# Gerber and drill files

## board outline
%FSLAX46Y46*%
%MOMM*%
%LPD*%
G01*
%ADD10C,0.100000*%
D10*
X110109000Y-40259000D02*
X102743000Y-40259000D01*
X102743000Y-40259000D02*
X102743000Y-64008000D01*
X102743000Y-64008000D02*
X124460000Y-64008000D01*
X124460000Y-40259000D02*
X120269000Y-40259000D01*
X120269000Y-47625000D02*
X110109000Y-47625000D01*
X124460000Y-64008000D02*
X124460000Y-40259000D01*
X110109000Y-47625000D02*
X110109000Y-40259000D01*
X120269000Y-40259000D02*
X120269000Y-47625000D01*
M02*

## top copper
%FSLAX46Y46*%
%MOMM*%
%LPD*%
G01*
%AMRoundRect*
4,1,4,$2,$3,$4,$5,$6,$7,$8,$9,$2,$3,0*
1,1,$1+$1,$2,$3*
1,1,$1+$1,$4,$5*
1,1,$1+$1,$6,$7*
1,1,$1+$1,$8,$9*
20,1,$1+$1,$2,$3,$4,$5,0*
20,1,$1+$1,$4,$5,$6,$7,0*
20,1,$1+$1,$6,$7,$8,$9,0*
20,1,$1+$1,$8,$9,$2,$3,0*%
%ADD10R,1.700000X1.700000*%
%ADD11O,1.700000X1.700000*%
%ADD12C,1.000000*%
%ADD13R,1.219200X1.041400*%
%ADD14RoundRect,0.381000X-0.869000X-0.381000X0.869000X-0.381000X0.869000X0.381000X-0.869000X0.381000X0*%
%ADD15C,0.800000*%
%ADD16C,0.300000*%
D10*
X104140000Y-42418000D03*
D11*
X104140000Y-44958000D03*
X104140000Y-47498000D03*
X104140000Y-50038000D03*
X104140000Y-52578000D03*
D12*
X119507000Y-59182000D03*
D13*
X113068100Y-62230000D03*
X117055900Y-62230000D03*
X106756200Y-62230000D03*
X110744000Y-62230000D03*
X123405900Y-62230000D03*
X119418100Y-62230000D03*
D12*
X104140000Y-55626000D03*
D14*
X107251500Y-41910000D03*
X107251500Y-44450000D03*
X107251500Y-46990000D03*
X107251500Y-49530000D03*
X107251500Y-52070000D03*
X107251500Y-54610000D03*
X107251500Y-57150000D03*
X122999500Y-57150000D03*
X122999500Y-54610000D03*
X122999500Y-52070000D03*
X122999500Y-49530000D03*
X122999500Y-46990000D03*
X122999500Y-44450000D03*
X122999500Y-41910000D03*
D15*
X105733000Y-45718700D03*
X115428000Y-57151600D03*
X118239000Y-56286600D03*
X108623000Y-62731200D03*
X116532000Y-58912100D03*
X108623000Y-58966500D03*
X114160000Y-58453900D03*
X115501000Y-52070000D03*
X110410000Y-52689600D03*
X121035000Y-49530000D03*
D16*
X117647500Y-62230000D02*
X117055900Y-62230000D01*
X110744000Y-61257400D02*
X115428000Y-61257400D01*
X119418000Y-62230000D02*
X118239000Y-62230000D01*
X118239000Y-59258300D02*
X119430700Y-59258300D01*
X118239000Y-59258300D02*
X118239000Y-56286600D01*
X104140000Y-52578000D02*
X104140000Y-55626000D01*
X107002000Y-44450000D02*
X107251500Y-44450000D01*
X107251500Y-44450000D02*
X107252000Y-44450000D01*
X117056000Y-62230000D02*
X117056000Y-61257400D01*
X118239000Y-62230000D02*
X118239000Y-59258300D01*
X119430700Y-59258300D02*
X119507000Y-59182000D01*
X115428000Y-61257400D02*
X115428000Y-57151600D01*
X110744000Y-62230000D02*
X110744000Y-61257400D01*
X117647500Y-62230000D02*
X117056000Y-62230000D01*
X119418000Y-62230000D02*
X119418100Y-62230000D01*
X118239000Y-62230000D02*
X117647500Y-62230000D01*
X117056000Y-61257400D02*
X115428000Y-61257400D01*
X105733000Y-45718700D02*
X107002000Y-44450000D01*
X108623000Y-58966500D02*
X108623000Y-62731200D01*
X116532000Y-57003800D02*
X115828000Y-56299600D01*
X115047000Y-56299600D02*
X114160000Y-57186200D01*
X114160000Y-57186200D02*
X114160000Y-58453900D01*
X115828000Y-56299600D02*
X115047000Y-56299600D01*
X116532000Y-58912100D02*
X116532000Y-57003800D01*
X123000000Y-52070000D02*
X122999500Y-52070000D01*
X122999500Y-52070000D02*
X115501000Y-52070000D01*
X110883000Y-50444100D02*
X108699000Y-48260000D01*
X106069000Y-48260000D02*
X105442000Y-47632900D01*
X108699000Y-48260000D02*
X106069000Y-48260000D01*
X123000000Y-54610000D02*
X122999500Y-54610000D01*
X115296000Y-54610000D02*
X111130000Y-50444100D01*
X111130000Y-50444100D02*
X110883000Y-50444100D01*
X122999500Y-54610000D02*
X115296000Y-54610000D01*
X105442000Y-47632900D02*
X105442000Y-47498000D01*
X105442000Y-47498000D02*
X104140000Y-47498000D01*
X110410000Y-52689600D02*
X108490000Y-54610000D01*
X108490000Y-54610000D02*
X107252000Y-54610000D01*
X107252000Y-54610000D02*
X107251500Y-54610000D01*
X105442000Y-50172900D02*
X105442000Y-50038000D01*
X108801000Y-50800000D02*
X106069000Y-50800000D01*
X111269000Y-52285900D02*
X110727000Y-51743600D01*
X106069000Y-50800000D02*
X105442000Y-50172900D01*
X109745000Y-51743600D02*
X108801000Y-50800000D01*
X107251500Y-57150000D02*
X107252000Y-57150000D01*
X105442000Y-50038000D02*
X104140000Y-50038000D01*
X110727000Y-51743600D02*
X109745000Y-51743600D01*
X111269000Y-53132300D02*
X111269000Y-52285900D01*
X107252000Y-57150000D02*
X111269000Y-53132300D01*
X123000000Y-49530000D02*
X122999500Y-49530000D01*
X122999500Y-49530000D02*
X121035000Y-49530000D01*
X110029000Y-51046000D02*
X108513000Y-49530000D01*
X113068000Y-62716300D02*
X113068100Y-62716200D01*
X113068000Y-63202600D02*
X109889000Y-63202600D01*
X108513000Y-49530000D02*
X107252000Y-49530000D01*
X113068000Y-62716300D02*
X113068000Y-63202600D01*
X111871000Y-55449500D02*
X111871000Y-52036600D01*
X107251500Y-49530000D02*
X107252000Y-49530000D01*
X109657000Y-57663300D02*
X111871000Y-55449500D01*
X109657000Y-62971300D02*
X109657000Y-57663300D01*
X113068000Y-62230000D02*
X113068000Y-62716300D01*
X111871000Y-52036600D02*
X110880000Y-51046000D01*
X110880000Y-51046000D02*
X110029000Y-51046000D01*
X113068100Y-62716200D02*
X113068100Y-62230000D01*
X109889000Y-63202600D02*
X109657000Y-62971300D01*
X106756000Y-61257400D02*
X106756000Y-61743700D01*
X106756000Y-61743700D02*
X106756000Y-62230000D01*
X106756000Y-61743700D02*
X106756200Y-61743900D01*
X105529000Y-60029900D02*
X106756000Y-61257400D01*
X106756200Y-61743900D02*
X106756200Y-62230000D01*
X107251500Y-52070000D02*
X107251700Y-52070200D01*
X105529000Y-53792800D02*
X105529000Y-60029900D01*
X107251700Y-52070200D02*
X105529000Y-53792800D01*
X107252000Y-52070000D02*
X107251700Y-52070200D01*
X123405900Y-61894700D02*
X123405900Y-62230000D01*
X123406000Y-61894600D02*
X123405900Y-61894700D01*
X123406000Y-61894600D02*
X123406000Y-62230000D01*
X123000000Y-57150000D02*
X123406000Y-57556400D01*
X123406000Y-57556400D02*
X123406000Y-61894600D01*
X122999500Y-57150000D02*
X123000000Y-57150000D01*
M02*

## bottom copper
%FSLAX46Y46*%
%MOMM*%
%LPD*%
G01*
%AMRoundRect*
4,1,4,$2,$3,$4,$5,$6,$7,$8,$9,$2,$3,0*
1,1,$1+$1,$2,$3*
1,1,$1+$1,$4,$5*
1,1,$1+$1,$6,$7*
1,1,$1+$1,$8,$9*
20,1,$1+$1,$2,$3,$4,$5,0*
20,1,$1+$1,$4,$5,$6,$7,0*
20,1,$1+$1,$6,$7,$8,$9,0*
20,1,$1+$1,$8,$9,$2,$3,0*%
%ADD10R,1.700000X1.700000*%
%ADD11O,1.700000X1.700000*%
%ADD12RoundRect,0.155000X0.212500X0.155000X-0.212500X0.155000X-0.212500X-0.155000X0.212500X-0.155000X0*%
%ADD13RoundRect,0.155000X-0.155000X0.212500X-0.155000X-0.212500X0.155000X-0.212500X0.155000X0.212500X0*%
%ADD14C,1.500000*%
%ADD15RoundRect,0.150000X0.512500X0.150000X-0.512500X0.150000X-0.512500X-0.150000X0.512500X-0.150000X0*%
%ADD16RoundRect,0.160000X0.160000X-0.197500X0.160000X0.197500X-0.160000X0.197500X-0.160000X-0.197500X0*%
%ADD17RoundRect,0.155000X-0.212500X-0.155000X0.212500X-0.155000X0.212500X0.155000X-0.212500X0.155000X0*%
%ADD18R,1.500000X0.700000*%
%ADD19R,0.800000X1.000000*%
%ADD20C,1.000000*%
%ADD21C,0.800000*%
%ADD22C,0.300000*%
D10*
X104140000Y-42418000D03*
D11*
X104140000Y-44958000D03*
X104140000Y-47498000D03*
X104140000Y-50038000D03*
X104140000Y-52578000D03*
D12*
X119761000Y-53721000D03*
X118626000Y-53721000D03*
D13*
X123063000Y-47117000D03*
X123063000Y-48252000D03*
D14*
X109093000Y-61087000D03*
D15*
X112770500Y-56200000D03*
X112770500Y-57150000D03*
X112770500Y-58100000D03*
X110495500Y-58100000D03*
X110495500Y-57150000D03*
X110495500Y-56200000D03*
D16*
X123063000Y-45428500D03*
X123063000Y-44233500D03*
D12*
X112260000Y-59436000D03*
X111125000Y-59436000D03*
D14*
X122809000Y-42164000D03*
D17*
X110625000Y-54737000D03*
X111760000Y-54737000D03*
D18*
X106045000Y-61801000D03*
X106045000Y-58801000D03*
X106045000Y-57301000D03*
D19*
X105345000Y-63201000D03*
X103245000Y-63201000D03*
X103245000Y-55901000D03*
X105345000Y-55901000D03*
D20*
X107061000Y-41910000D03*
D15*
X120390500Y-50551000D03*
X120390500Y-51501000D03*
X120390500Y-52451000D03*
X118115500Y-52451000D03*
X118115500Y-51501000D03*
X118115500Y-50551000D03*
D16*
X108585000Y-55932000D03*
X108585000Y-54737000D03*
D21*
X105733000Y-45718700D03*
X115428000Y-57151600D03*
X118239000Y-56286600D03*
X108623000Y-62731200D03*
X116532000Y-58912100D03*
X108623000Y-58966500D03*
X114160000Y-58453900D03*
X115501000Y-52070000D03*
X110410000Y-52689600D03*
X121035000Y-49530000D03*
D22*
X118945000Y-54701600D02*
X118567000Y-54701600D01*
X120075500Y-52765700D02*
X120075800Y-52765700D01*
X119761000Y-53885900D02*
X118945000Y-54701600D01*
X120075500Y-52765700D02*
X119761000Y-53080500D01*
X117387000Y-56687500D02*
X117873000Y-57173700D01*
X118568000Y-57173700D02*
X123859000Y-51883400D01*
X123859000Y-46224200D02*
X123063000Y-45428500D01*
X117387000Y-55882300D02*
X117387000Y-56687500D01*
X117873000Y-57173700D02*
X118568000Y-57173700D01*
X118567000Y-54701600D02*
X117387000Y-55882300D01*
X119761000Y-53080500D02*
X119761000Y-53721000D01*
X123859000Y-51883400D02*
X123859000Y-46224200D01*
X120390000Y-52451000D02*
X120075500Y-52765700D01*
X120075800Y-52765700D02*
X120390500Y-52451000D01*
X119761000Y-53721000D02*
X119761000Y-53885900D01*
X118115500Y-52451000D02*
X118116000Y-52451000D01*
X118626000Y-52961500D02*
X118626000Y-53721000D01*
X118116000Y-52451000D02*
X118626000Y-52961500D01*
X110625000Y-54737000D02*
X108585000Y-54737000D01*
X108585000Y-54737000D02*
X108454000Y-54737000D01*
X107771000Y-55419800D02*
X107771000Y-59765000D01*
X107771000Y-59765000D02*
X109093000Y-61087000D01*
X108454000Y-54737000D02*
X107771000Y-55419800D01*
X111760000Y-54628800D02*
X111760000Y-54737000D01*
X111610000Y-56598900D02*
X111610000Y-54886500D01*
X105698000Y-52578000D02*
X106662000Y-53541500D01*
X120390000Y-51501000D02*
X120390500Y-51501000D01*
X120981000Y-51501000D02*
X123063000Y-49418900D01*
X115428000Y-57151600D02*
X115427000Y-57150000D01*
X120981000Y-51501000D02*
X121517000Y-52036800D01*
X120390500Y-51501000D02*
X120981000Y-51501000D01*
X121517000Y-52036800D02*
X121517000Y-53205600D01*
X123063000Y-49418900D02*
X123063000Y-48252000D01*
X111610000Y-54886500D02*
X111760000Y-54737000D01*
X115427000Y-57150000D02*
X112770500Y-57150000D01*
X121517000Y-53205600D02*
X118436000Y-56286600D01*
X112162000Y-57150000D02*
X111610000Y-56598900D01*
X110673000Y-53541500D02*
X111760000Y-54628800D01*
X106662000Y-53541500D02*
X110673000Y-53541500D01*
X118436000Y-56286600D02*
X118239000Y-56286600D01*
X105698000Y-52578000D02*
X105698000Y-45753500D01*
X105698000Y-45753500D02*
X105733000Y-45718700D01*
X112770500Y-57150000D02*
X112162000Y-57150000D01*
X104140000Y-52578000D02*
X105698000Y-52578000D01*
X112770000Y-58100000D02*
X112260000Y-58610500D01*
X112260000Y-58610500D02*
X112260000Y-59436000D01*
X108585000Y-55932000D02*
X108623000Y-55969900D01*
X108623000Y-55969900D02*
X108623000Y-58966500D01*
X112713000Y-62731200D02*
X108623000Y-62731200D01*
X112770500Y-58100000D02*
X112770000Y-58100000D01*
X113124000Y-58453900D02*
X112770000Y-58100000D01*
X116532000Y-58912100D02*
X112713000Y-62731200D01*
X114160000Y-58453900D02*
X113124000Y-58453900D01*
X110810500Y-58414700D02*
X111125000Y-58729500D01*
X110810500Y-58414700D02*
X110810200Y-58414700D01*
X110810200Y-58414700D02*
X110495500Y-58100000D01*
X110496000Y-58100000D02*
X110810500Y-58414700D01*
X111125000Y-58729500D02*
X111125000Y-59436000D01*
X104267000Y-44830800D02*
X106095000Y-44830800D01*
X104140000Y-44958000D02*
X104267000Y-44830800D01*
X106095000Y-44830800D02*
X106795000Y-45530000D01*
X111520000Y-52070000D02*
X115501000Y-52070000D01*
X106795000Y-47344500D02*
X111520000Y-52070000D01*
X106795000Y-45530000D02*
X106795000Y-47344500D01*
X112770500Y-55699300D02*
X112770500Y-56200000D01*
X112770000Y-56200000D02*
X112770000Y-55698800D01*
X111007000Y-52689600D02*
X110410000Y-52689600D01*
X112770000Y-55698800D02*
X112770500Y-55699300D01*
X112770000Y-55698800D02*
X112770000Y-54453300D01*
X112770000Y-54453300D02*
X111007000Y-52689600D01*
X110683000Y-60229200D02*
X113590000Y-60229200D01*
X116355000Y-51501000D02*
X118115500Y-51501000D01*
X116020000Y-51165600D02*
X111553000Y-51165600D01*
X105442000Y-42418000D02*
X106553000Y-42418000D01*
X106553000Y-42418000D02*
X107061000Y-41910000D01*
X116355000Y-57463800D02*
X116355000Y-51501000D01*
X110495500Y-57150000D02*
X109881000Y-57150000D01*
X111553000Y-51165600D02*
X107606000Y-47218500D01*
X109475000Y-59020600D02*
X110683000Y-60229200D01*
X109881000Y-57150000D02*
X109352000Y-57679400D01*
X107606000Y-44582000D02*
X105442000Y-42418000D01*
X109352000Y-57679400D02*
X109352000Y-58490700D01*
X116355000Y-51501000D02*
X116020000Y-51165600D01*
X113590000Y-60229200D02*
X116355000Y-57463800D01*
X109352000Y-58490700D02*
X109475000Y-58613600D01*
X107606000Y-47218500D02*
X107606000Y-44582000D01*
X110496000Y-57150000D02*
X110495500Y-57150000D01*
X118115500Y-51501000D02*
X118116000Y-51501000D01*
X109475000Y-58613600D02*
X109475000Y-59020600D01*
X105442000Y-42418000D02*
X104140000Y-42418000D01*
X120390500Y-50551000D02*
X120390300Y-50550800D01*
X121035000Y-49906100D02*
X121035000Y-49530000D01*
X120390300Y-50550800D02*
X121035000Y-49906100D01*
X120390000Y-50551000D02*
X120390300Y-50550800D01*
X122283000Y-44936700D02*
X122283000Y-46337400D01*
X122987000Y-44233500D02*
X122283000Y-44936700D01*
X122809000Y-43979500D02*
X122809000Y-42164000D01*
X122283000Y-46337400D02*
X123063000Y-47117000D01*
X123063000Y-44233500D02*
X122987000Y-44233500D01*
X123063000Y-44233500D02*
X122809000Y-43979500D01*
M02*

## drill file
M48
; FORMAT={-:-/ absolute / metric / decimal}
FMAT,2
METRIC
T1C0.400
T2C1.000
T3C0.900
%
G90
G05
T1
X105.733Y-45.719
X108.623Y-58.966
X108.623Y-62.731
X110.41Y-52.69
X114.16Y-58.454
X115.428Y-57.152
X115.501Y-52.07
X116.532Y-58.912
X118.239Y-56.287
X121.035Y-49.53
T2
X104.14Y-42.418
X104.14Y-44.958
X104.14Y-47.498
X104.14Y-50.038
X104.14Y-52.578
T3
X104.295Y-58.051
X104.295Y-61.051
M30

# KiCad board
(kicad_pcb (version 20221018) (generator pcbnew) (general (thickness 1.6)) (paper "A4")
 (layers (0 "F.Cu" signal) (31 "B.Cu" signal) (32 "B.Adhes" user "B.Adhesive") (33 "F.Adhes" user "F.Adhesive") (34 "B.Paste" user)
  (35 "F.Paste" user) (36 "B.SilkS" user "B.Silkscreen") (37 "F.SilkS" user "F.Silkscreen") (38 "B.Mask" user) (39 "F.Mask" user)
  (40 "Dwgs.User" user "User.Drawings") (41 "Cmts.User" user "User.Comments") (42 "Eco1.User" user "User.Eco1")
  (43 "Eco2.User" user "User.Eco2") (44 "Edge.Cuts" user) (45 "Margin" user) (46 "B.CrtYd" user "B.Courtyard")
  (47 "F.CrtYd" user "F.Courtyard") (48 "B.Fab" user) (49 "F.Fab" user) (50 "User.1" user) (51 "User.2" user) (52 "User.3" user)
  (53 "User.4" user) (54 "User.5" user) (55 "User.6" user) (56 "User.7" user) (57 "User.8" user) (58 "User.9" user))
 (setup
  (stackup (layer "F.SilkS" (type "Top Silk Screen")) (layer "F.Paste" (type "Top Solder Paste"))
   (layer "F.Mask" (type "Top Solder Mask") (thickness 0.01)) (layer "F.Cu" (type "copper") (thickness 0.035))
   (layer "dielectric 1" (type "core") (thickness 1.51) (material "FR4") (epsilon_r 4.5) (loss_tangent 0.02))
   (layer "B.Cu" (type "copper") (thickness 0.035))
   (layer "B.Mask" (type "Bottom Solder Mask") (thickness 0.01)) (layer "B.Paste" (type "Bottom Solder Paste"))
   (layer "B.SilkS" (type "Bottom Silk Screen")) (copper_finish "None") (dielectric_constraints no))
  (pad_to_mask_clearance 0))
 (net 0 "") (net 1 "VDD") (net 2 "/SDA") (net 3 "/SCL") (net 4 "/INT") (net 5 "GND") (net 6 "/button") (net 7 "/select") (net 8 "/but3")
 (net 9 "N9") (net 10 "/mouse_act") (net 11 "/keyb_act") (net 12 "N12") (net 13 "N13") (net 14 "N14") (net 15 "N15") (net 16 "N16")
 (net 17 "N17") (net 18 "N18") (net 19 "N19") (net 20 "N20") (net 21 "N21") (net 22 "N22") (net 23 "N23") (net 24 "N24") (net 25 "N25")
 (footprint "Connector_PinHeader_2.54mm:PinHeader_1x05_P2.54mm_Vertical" (layer "F.Cu") (at 104.14 42.418)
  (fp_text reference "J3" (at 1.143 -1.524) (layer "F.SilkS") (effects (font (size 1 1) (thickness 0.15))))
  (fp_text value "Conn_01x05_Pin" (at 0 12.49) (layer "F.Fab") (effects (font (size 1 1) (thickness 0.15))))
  (pad "1" thru_hole rect (at 0 0) (size 1.7 1.7) (drill 1) (layers "*.Cu" "*.Mask") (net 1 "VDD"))
  (pad "2" thru_hole oval (at 0 2.54) (size 1.7 1.7) (drill 1) (layers "*.Cu" "*.Mask") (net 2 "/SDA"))
  (pad "3" thru_hole oval (at 0 5.08) (size 1.7 1.7) (drill 1) (layers "*.Cu" "*.Mask") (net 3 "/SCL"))
  (pad "4" thru_hole oval (at 0 7.62) (size 1.7 1.7) (drill 1) (layers "*.Cu" "*.Mask") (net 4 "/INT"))
  (pad "5" thru_hole oval (at 0 10.16) (size 1.7 1.7) (drill 1) (layers "*.Cu" "*.Mask") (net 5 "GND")))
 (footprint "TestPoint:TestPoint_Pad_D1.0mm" (layer "F.Cu") (at 119.507 59.182)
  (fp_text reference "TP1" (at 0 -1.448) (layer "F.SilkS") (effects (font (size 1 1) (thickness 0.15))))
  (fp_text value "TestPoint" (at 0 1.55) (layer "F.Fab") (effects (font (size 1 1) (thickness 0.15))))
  (pad "1" smd circle (at 0 0) (size 1 1) (layers "F.Cu" "F.Mask") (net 5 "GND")))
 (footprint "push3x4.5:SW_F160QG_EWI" (layer "F.Cu") (at 115.062 62.23)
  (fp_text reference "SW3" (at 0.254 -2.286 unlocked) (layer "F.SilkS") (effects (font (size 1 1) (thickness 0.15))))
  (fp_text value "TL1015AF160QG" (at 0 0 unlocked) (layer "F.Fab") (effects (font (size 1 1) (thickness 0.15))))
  (pad "1" smd rect (at -1.9939 0) (size 1.2192 1.0414) (layers "F.Cu" "F.Paste" "F.Mask") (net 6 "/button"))
  (pad "2" smd rect (at 1.9939 0) (size 1.2192 1.0414) (layers "F.Cu" "F.Paste" "F.Mask") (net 5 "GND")))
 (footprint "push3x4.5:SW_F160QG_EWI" (layer "F.Cu") (at 108.7501 62.23)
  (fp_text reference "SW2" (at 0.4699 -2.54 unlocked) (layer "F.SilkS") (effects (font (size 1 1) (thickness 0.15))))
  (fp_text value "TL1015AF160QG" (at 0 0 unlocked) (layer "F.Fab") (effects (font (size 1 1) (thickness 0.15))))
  (pad "1" smd rect (at -1.9939 0) (size 1.2192 1.0414) (layers "F.Cu" "F.Paste" "F.Mask") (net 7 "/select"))
  (pad "2" smd rect (at 1.9939 0) (size 1.2192 1.0414) (layers "F.Cu" "F.Paste" "F.Mask") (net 5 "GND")))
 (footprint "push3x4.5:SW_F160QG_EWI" (layer "F.Cu") (at 121.412 62.23 180)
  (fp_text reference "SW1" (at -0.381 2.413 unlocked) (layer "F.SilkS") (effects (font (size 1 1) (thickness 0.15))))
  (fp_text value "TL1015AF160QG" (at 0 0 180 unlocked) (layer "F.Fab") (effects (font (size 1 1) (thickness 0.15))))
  (pad "1" smd rect (at -1.9939 0 180) (size 1.2192 1.0414) (layers "F.Cu" "F.Paste" "F.Mask") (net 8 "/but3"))
  (pad "2" smd rect (at 1.9939 0 180) (size 1.2192 1.0414) (layers "F.Cu" "F.Paste" "F.Mask") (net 5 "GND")))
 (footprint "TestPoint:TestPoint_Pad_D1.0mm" (layer "F.Cu") (at 104.14 55.626)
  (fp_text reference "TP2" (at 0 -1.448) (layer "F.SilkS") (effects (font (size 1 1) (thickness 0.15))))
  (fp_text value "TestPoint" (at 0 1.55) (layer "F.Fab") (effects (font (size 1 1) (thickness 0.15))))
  (pad "1" smd circle (at 0 0) (size 1 1) (layers "F.Cu" "F.Mask") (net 5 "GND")))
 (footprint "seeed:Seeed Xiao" (layer "F.Cu") (at 109.0295 41.91)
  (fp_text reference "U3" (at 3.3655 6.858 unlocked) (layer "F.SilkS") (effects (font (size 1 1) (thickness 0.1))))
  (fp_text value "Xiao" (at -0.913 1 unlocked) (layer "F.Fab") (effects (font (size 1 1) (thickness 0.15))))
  (pad "1" smd roundrect (at -1.778 0) (size 2.5 1.524) (layers "F.Cu" "F.Paste" "F.Mask") (roundrect_rratio 0.25) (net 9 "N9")
   (thermal_bridge_angle 45))
  (pad "2" smd roundrect (at -1.778 2.54) (size 2.5 1.524) (layers "F.Cu" "F.Paste" "F.Mask") (roundrect_rratio 0.25) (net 5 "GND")
   (thermal_bridge_angle 45))
  (pad "3" smd roundrect (at -1.778 5.08) (size 2.5 1.524) (layers "F.Cu" "F.Paste" "F.Mask") (roundrect_rratio 0.25) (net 1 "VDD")
   (thermal_bridge_angle 45))
  (pad "4" smd roundrect (at -1.778 7.62) (size 2.5 1.524) (layers "F.Cu" "F.Paste" "F.Mask") (roundrect_rratio 0.25) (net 6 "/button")
   (thermal_bridge_angle 45))
  (pad "5" smd roundrect (at -1.778 10.16) (size 2.5 1.524) (layers "F.Cu" "F.Paste" "F.Mask") (roundrect_rratio 0.25) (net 7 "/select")
   (thermal_bridge_angle 45))
  (pad "6" smd roundrect (at -1.778 12.7) (size 2.5 1.524) (layers "F.Cu" "F.Paste" "F.Mask") (roundrect_rratio 0.25) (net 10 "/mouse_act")
   (thermal_bridge_angle 45))
  (pad "7" smd roundrect (at -1.778 15.24) (size 2.5 1.524) (layers "F.Cu" "F.Paste" "F.Mask") (roundrect_rratio 0.25) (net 4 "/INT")
   (thermal_bridge_angle 45))
  (pad "8" smd roundrect (at 13.97 15.24) (size 2.5 1.524) (layers "F.Cu" "F.Paste" "F.Mask") (roundrect_rratio 0.25) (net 8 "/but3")
   (thermal_bridge_angle 45))
  (pad "9" smd roundrect (at 13.97 12.7) (size 2.5 1.524) (layers "F.Cu" "F.Paste" "F.Mask") (roundrect_rratio 0.25) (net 3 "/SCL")
   (thermal_bridge_angle 45))
  (pad "10" smd roundrect (at 13.97 10.16) (size 2.5 1.524) (layers "F.Cu" "F.Paste" "F.Mask") (roundrect_rratio 0.25) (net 2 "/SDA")
   (thermal_bridge_angle 45))
  (pad "11" smd roundrect (at 13.97 7.62) (size 2.5 1.524) (layers "F.Cu" "F.Paste" "F.Mask") (roundrect_rratio 0.25) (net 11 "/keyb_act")
   (thermal_bridge_angle 45))
  (pad "12" smd roundrect (at 13.97 5.08) (size 2.5 1.524) (layers "F.Cu" "F.Paste" "F.Mask") (roundrect_rratio 0.25) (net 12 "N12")
   (thermal_bridge_angle 45))
  (pad "13" smd roundrect (at 13.97 2.54) (size 2.5 1.524) (layers "F.Cu" "F.Paste" "F.Mask") (roundrect_rratio 0.25) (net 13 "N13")
   (thermal_bridge_angle 45))
  (pad "14" smd roundrect (at 13.97 0) (size 2.5 1.524) (layers "F.Cu" "F.Paste" "F.Mask") (roundrect_rratio 0.25) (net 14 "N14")
   (thermal_bridge_angle 45)))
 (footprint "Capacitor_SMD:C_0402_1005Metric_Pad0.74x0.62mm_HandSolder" (layer "B.Cu") (at 119.1935 53.721 180)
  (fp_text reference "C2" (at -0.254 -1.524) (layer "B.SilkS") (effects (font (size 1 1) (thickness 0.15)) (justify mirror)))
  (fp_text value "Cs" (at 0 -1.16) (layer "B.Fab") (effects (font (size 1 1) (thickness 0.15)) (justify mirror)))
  (pad "1" smd roundrect (at -0.5675 0 180) (size 0.735 0.62) (layers "B.Cu" "B.Paste" "B.Mask") (roundrect_rratio 0.25) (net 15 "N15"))
  (pad "2" smd roundrect (at 0.5675 0 180) (size 0.735 0.62) (layers "B.Cu" "B.Paste" "B.Mask") (roundrect_rratio 0.25) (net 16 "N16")))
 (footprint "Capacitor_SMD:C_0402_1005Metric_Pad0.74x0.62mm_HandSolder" (layer "B.Cu") (at 123.063 47.6845 -90)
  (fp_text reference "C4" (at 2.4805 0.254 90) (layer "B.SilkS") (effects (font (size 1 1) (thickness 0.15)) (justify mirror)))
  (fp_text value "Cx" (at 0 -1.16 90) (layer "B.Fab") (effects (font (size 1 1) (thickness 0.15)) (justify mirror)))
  (pad "1" smd roundrect (at -0.5675 0 270) (size 0.735 0.62) (layers "B.Cu" "B.Paste" "B.Mask") (roundrect_rratio 0.25) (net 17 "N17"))
  (pad "2" smd roundrect (at 0.5675 0 270) (size 0.735 0.62) (layers "B.Cu" "B.Paste" "B.Mask") (roundrect_rratio 0.25) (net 5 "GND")))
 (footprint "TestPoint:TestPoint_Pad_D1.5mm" (layer "B.Cu") (at 109.093 61.087 180)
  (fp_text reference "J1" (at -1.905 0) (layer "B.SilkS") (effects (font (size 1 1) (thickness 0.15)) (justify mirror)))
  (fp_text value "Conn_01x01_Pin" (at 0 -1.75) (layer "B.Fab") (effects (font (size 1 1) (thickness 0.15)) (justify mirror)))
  (pad "1" smd circle (at 0 0 180) (size 1.5 1.5) (layers "B.Cu" "B.Mask") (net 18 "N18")))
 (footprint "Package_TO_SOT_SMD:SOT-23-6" (layer "B.Cu") (at 111.633 57.15 180)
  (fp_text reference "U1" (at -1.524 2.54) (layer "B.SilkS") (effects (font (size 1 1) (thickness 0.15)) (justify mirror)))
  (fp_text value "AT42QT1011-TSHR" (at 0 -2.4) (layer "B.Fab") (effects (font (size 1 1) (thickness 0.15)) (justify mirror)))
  (pad "1" smd roundrect (at -1.1375 0.95 180) (size 1.325 0.6) (layers "B.Cu" "B.Paste" "B.Mask") (roundrect_rratio 0.25)
   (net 10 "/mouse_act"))
  (pad "2" smd roundrect (at -1.1375 0 180) (size 1.325 0.6) (layers "B.Cu" "B.Paste" "B.Mask") (roundrect_rratio 0.25) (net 5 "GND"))
  (pad "3" smd roundrect (at -1.1375 -0.95 180) (size 1.325 0.6) (layers "B.Cu" "B.Paste" "B.Mask") (roundrect_rratio 0.25) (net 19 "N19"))
  (pad "4" smd roundrect (at 1.1375 -0.95 180) (size 1.325 0.6) (layers "B.Cu" "B.Paste" "B.Mask") (roundrect_rratio 0.25) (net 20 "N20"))
  (pad "5" smd roundrect (at 1.1375 0 180) (size 1.325 0.6) (layers "B.Cu" "B.Paste" "B.Mask") (roundrect_rratio 0.25) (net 1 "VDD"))
  (pad "6" smd roundrect (at 1.1375 0.95 180) (size 1.325 0.6) (layers "B.Cu" "B.Paste" "B.Mask") (roundrect_rratio 0.25) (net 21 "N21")))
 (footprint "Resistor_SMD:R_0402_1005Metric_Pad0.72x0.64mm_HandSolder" (layer "B.Cu") (at 123.063 44.831 90)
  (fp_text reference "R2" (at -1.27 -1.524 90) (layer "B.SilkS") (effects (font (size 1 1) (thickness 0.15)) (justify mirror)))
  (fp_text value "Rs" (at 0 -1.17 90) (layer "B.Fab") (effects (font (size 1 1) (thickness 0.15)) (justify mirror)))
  (pad "1" smd roundrect (at -0.5975 0 90) (size 0.715 0.64) (layers "B.Cu" "B.Paste" "B.Mask") (roundrect_rratio 0.25) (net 15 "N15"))
  (pad "2" smd roundrect (at 0.5975 0 90) (size 0.715 0.64) (layers "B.Cu" "B.Paste" "B.Mask") (roundrect_rratio 0.25) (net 17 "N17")))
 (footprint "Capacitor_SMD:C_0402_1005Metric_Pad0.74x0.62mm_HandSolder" (layer "B.Cu") (at 111.6925 59.436 180)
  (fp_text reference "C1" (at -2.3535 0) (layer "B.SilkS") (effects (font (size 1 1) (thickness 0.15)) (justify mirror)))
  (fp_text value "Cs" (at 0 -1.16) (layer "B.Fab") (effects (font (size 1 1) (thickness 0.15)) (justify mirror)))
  (pad "1" smd roundrect (at -0.5675 0 180) (size 0.735 0.62) (layers "B.Cu" "B.Paste" "B.Mask") (roundrect_rratio 0.25) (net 19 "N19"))
  (pad "2" smd roundrect (at 0.5675 0 180) (size 0.735 0.62) (layers "B.Cu" "B.Paste" "B.Mask") (roundrect_rratio 0.25) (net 20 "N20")))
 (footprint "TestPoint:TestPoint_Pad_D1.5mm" (layer "B.Cu") (at 122.809 42.164 180)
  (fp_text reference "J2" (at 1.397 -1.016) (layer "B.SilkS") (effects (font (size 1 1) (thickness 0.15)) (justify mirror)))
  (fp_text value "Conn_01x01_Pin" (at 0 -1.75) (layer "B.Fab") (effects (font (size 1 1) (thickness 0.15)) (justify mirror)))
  (pad "1" smd circle (at 0 0 180) (size 1.5 1.5) (layers "B.Cu" "B.Mask") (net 17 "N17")))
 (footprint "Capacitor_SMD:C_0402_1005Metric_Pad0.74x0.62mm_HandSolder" (layer "B.Cu") (at 111.1925 54.737)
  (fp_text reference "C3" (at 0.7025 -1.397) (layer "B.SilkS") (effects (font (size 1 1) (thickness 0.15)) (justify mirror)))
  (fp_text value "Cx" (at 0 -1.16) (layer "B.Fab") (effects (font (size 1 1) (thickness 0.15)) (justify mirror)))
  (pad "1" smd roundrect (at -0.5675 0) (size 0.735 0.62) (layers "B.Cu" "B.Paste" "B.Mask") (roundrect_rratio 0.25) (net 18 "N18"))
  (pad "2" smd roundrect (at 0.5675 0) (size 0.735 0.62) (layers "B.Cu" "B.Paste" "B.Mask") (roundrect_rratio 0.25) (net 5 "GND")))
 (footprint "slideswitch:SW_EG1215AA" (layer "B.Cu") (at 104.295 59.551 90)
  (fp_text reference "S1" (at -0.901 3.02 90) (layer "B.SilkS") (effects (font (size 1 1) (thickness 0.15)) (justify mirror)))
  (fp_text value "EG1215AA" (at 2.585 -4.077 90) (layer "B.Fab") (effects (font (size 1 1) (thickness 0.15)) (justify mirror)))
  (pad "" np_thru_hole circle (at -1.5 0 90) (size 0.9 0.9) (drill 0.9) (layers "*.Cu" "*.Mask"))
  (pad "" np_thru_hole circle (at 1.5 0 90) (size 0.9 0.9) (drill 0.9) (layers "*.Cu" "*.Mask"))
  (pad "1" smd rect (at -2.25 1.75 90) (size 0.7 1.5) (layers "B.Cu" "B.Paste" "B.Mask") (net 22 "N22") (solder_mask_margin 0.102))
  (pad "2" smd rect (at 0.75 1.75 90) (size 0.7 1.5) (layers "B.Cu" "B.Paste" "B.Mask") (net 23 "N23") (solder_mask_margin 0.102))
  (pad "3" smd rect (at 2.25 1.75 90) (size 0.7 1.5) (layers "B.Cu" "B.Paste" "B.Mask") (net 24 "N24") (solder_mask_margin 0.102))
  (pad "S1" smd rect (at -3.65 1.05 90) (size 1 0.8) (layers "B.Cu" "B.Paste" "B.Mask") (solder_mask_margin 0.102))
  (pad "S2" smd rect (at -3.65 -1.05 90) (size 1 0.8) (layers "B.Cu" "B.Paste" "B.Mask") (solder_mask_margin 0.102))
  (pad "S3" smd rect (at 3.65 -1.05 90) (size 1 0.8) (layers "B.Cu" "B.Paste" "B.Mask") (solder_mask_margin 0.102))
  (pad "S4" smd rect (at 3.65 1.05 90) (size 1 0.8) (layers "B.Cu" "B.Paste" "B.Mask") (solder_mask_margin 0.102)))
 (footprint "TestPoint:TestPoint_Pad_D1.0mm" (layer "B.Cu") (at 107.061 41.91 180)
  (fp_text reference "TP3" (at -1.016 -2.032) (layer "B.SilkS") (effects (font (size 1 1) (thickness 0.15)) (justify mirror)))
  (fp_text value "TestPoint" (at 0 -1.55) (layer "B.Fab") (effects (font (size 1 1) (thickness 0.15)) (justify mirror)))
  (pad "1" smd circle (at 0 0 180) (size 1 1) (layers "B.Cu" "B.Mask") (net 1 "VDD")))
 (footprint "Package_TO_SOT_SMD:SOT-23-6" (layer "B.Cu") (at 119.253 51.501 180)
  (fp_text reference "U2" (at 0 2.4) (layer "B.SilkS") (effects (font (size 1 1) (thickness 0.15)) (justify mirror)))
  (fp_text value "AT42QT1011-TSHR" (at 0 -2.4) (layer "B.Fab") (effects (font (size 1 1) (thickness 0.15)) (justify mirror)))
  (pad "1" smd roundrect (at -1.1375 0.95 180) (size 1.325 0.6) (layers "B.Cu" "B.Paste" "B.Mask") (roundrect_rratio 0.25)
   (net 11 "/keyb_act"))
  (pad "2" smd roundrect (at -1.1375 0 180) (size 1.325 0.6) (layers "B.Cu" "B.Paste" "B.Mask") (roundrect_rratio 0.25) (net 5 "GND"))
  (pad "3" smd roundrect (at -1.1375 -0.95 180) (size 1.325 0.6) (layers "B.Cu" "B.Paste" "B.Mask") (roundrect_rratio 0.25) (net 15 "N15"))
  (pad "4" smd roundrect (at 1.1375 -0.95 180) (size 1.325 0.6) (layers "B.Cu" "B.Paste" "B.Mask") (roundrect_rratio 0.25) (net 16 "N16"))
  (pad "5" smd roundrect (at 1.1375 0 180) (size 1.325 0.6) (layers "B.Cu" "B.Paste" "B.Mask") (roundrect_rratio 0.25) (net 1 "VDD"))
  (pad "6" smd roundrect (at 1.1375 0.95 180) (size 1.325 0.6) (layers "B.Cu" "B.Paste" "B.Mask") (roundrect_rratio 0.25) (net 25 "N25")))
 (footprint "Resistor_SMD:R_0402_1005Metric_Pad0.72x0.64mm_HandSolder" (layer "B.Cu") (at 108.585 55.3345 90)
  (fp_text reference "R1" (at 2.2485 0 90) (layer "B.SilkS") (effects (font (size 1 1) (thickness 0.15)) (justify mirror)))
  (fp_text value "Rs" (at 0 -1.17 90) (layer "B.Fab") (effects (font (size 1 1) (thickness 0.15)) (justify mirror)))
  (pad "1" smd roundrect (at -0.5975 0 90) (size 0.715 0.64) (layers "B.Cu" "B.Paste" "B.Mask") (roundrect_rratio 0.25) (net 19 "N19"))
  (pad "2" smd roundrect (at 0.5975 0 90) (size 0.715 0.64) (layers "B.Cu" "B.Paste" "B.Mask") (roundrect_rratio 0.25) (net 18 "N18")))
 (gr_line (start 110.109 40.259) (end 102.743 40.259) (stroke (width 0.1) (type default)) (layer "Edge.Cuts"))
 (gr_line (start 102.743 40.259) (end 102.743 64.008) (stroke (width 0.1) (type default)) (layer "Edge.Cuts"))
 (gr_line (start 102.743 64.008) (end 124.46 64.008) (stroke (width 0.1) (type default)) (layer "Edge.Cuts"))
 (gr_line (start 124.46 40.259) (end 120.269 40.259) (stroke (width 0.1) (type default)) (layer "Edge.Cuts"))
 (gr_line (start 120.269 47.625) (end 110.109 47.625) (stroke (width 0.1) (type default)) (layer "Edge.Cuts"))
 (gr_line (start 124.46 64.008) (end 124.46 40.259) (stroke (width 0.1) (type default)) (layer "Edge.Cuts"))
 (gr_line (start 110.109 47.625) (end 110.109 40.259) (stroke (width 0.1) (type default)) (layer "Edge.Cuts"))
 (gr_line (start 120.269 40.259) (end 120.269 47.625) (stroke (width 0.1) (type default)) (layer "Edge.Cuts"))
 (segment (start 118.945 54.7016) (end 118.567 54.7016) (width 0.3) (layer "B.Cu") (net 15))
 (segment (start 120.0755 52.7657) (end 120.0758 52.7657) (width 0.3) (layer "B.Cu") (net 15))
 (segment (start 119.761 53.8859) (end 118.945 54.7016) (width 0.3) (layer "B.Cu") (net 15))
 (segment (start 120.0755 52.7657) (end 119.761 53.0805) (width 0.3) (layer "B.Cu") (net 15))
 (segment (start 117.387 56.6875) (end 117.873 57.1737) (width 0.3) (layer "B.Cu") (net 15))
 (segment (start 118.568 57.1737) (end 123.859 51.8834) (width 0.3) (layer "B.Cu") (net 15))
 (segment (start 123.859 46.2242) (end 123.063 45.4285) (width 0.3) (layer "B.Cu") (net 15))
 (segment (start 117.387 55.8823) (end 117.387 56.6875) (width 0.3) (layer "B.Cu") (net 15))
 (segment (start 117.873 57.1737) (end 118.568 57.1737) (width 0.3) (layer "B.Cu") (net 15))
 (segment (start 118.567 54.7016) (end 117.387 55.8823) (width 0.3) (layer "B.Cu") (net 15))
 (segment (start 119.761 53.0805) (end 119.761 53.721) (width 0.3) (layer "B.Cu") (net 15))
 (segment (start 123.859 51.8834) (end 123.859 46.2242) (width 0.3) (layer "B.Cu") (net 15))
 (segment (start 120.39 52.451) (end 120.0755 52.7657) (width 0.3) (layer "B.Cu") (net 15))
 (segment (start 120.0758 52.7657) (end 120.3905 52.451) (width 0.3) (layer "B.Cu") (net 15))
 (segment (start 119.761 53.721) (end 119.761 53.8859) (width 0.3) (layer "B.Cu") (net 15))
 (segment (start 118.1155 52.451) (end 118.116 52.451) (width 0.3) (layer "B.Cu") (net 16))
 (segment (start 118.626 52.9615) (end 118.626 53.721) (width 0.3) (layer "B.Cu") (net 16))
 (segment (start 118.116 52.451) (end 118.626 52.9615) (width 0.3) (layer "B.Cu") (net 16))
 (segment (start 110.625 54.737) (end 108.585 54.737) (width 0.3) (layer "B.Cu") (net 18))
 (segment (start 108.585 54.737) (end 108.454 54.737) (width 0.3) (layer "B.Cu") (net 18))
 (segment (start 107.771 55.4198) (end 107.771 59.765) (width 0.3) (layer "B.Cu") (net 18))
 (segment (start 107.771 59.765) (end 109.093 61.087) (width 0.3) (layer "B.Cu") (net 18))
 (segment (start 108.454 54.737) (end 107.771 55.4198) (width 0.3) (layer "B.Cu") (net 18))
 (segment (start 117.6475 62.23) (end 117.0559 62.23) (width 0.3) (layer "F.Cu") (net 5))
 (segment (start 110.744 61.2574) (end 115.428 61.2574) (width 0.3) (layer "F.Cu") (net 5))
 (segment (start 119.418 62.23) (end 118.239 62.23) (width 0.3) (layer "F.Cu") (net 5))
 (segment (start 118.239 59.2583) (end 119.4307 59.2583) (width 0.3) (layer "F.Cu") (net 5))
 (segment (start 118.239 59.2583) (end 118.239 56.2866) (width 0.3) (layer "F.Cu") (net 5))
 (segment (start 104.14 52.578) (end 104.14 55.626) (width 0.3) (layer "F.Cu") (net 5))
 (segment (start 107.002 44.45) (end 107.2515 44.45) (width 0.3) (layer "F.Cu") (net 5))
 (segment (start 107.2515 44.45) (end 107.252 44.45) (width 0.3) (layer "F.Cu") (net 5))
 (segment (start 117.056 62.23) (end 117.056 61.2574) (width 0.3) (layer "F.Cu") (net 5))
 (segment (start 118.239 62.23) (end 118.239 59.2583) (width 0.3) (layer "F.Cu") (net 5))
 (segment (start 119.4307 59.2583) (end 119.507 59.182) (width 0.3) (layer "F.Cu") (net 5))
 (segment (start 115.428 61.2574) (end 115.428 57.1516) (width 0.3) (layer "F.Cu") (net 5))
 (segment (start 110.744 62.23) (end 110.744 61.2574) (width 0.3) (layer "F.Cu") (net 5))
 (segment (start 117.6475 62.23) (end 117.056 62.23) (width 0.3) (layer "F.Cu") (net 5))
 (segment (start 119.418 62.23) (end 119.4181 62.23) (width 0.3) (layer "F.Cu") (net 5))
 (segment (start 118.239 62.23) (end 117.6475 62.23) (width 0.3) (layer "F.Cu") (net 5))
 (segment (start 117.056 61.2574) (end 115.428 61.2574) (width 0.3) (layer "F.Cu") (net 5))
 (segment (start 105.733 45.7187) (end 107.002 44.45) (width 0.3) (layer "F.Cu") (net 5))
 (via (at 105.733 45.7187) (size 0.8) (drill 0.4) (layers "F.Cu" "B.Cu") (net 5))
 (via (at 115.428 57.1516) (size 0.8) (drill 0.4) (layers "F.Cu" "B.Cu") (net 5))
 (via (at 118.239 56.2866) (size 0.8) (drill 0.4) (layers "F.Cu" "B.Cu") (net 5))
 (segment (start 111.76 54.6288) (end 111.76 54.737) (width 0.3) (layer "B.Cu") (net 5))
 (segment (start 111.61 56.5989) (end 111.61 54.8865) (width 0.3) (layer "B.Cu") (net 5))
 (segment (start 105.698 52.578) (end 106.662 53.5415) (width 0.3) (layer "B.Cu") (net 5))
 (segment (start 120.39 51.501) (end 120.3905 51.501) (width 0.3) (layer "B.Cu") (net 5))
 (segment (start 120.981 51.501) (end 123.063 49.4189) (width 0.3) (layer "B.Cu") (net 5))
 (segment (start 115.428 57.1516) (end 115.427 57.15) (width 0.3) (layer "B.Cu") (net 5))
 (segment (start 120.981 51.501) (end 121.517 52.0368) (width 0.3) (layer "B.Cu") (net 5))
 (segment (start 120.3905 51.501) (end 120.981 51.501) (width 0.3) (layer "B.Cu") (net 5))
 (segment (start 121.517 52.0368) (end 121.517 53.2056) (width 0.3) (layer "B.Cu") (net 5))
 (segment (start 123.063 49.4189) (end 123.063 48.252) (width 0.3) (layer "B.Cu") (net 5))
 (segment (start 111.61 54.8865) (end 111.76 54.737) (width 0.3) (layer "B.Cu") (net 5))
 (segment (start 115.427 57.15) (end 112.7705 57.15) (width 0.3) (layer "B.Cu") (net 5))
 (segment (start 121.517 53.2056) (end 118.436 56.2866) (width 0.3) (layer "B.Cu") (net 5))
 (segment (start 112.162 57.15) (end 111.61 56.5989) (width 0.3) (layer "B.Cu") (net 5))
 (segment (start 110.673 53.5415) (end 111.76 54.6288) (width 0.3) (layer "B.Cu") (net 5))
 (segment (start 106.662 53.5415) (end 110.673 53.5415) (width 0.3) (layer "B.Cu") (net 5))
 (segment (start 118.436 56.2866) (end 118.239 56.2866) (width 0.3) (layer "B.Cu") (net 5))
 (segment (start 105.698 52.578) (end 105.698 45.7535) (width 0.3) (layer "B.Cu") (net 5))
 (segment (start 105.698 45.7535) (end 105.733 45.7187) (width 0.3) (layer "B.Cu") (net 5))
 (segment (start 112.7705 57.15) (end 112.162 57.15) (width 0.3) (layer "B.Cu") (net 5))
 (segment (start 104.14 52.578) (end 105.698 52.578) (width 0.3) (layer "B.Cu") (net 5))
 (segment (start 108.623 58.9665) (end 108.623 62.7312) (width 0.3) (layer "F.Cu") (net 19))
 (segment (start 116.532 57.0038) (end 115.828 56.2996) (width 0.3) (layer "F.Cu") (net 19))
 (segment (start 115.047 56.2996) (end 114.16 57.1862) (width 0.3) (layer "F.Cu") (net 19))
 (segment (start 114.16 57.1862) (end 114.16 58.4539) (width 0.3) (layer "F.Cu") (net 19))
 (segment (start 115.828 56.2996) (end 115.047 56.2996) (width 0.3) (layer "F.Cu") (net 19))
 (segment (start 116.532 58.9121) (end 116.532 57.0038) (width 0.3) (layer "F.Cu") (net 19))
 (via (at 108.623 62.7312) (size 0.8) (drill 0.4) (layers "F.Cu" "B.Cu") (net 19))
 (via (at 116.532 58.9121) (size 0.8) (drill 0.4) (layers "F.Cu" "B.Cu") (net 19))
 (via (at 108.623 58.9665) (size 0.8) (drill 0.4) (layers "F.Cu" "B.Cu") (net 19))
 (via (at 114.16 58.4539) (size 0.8) (drill 0.4) (layers "F.Cu" "B.Cu") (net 19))
 (segment (start 112.77 58.1) (end 112.26 58.6105) (width 0.3) (layer "B.Cu") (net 19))
 (segment (start 112.26 58.6105) (end 112.26 59.436) (width 0.3) (layer "B.Cu") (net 19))
 (segment (start 108.585 55.932) (end 108.623 55.9699) (width 0.3) (layer "B.Cu") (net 19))
 (segment (start 108.623 55.9699) (end 108.623 58.9665) (width 0.3) (layer "B.Cu") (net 19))
 (segment (start 112.713 62.7312) (end 108.623 62.7312) (width 0.3) (layer "B.Cu") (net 19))
 (segment (start 112.7705 58.1) (end 112.77 58.1) (width 0.3) (layer "B.Cu") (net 19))
 (segment (start 113.124 58.4539) (end 112.77 58.1) (width 0.3) (layer "B.Cu") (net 19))
 (segment (start 116.532 58.9121) (end 112.713 62.7312) (width 0.3) (layer "B.Cu") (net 19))
 (segment (start 114.16 58.4539) (end 113.124 58.4539) (width 0.3) (layer "B.Cu") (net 19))
 (segment (start 110.8105 58.4147) (end 111.125 58.7295) (width 0.3) (layer "B.Cu") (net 20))
 (segment (start 110.8105 58.4147) (end 110.8102 58.4147) (width 0.3) (layer "B.Cu") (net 20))
 (segment (start 110.8102 58.4147) (end 110.4955 58.1) (width 0.3) (layer "B.Cu") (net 20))
 (segment (start 110.496 58.1) (end 110.8105 58.4147) (width 0.3) (layer "B.Cu") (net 20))
 (segment (start 111.125 58.7295) (end 111.125 59.436) (width 0.3) (layer "B.Cu") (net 20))
 (segment (start 123 52.07) (end 122.9995 52.07) (width 0.3) (layer "F.Cu") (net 2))
 (segment (start 122.9995 52.07) (end 115.501 52.07) (width 0.3) (layer "F.Cu") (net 2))
 (via (at 115.501 52.07) (size 0.8) (drill 0.4) (layers "F.Cu" "B.Cu") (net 2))
 (segment (start 104.267 44.8308) (end 106.095 44.8308) (width 0.3) (layer "B.Cu") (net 2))
 (segment (start 104.14 44.958) (end 104.267 44.8308) (width 0.3) (layer "B.Cu") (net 2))
 (segment (start 106.095 44.8308) (end 106.795 45.53) (width 0.3) (layer "B.Cu") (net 2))
 (segment (start 111.52 52.07) (end 115.501 52.07) (width 0.3) (layer "B.Cu") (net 2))
 (segment (start 106.795 47.3445) (end 111.52 52.07) (width 0.3) (layer "B.Cu") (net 2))
 (segment (start 106.795 45.53) (end 106.795 47.3445) (width 0.3) (layer "B.Cu") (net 2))
 (segment (start 110.883 50.4441) (end 108.699 48.26) (width 0.3) (layer "F.Cu") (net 3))
 (segment (start 106.069 48.26) (end 105.442 47.6329) (width 0.3) (layer "F.Cu") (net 3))
 (segment (start 108.699 48.26) (end 106.069 48.26) (width 0.3) (layer "F.Cu") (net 3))
 (segment (start 123 54.61) (end 122.9995 54.61) (width 0.3) (layer "F.Cu") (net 3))
 (segment (start 115.296 54.61) (end 111.13 50.4441) (width 0.3) (layer "F.Cu") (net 3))
 (segment (start 111.13 50.4441) (end 110.883 50.4441) (width 0.3) (layer "F.Cu") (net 3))
 (segment (start 122.9995 54.61) (end 115.296 54.61) (width 0.3) (layer "F.Cu") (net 3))
 (segment (start 105.442 47.6329) (end 105.442 47.498) (width 0.3) (layer "F.Cu") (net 3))
 (segment (start 105.442 47.498) (end 104.14 47.498) (width 0.3) (layer "F.Cu") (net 3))
 (segment (start 110.41 52.6896) (end 108.49 54.61) (width 0.3) (layer "F.Cu") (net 10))
 (segment (start 108.49 54.61) (end 107.252 54.61) (width 0.3) (layer "F.Cu") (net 10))
 (segment (start 107.252 54.61) (end 107.2515 54.61) (width 0.3) (layer "F.Cu") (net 10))
 (via (at 110.41 52.6896) (size 0.8) (drill 0.4) (layers "F.Cu" "B.Cu") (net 10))
 (segment (start 112.7705 55.6993) (end 112.7705 56.2) (width 0.3) (layer "B.Cu") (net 10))
 (segment (start 112.77 56.2) (end 112.77 55.6988) (width 0.3) (layer "B.Cu") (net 10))
 (segment (start 111.007 52.6896) (end 110.41 52.6896) (width 0.3) (layer "B.Cu") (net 10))
 (segment (start 112.77 55.6988) (end 112.7705 55.6993) (width 0.3) (layer "B.Cu") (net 10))
 (segment (start 112.77 55.6988) (end 112.77 54.4533) (width 0.3) (layer "B.Cu") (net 10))
 (segment (start 112.77 54.4533) (end 111.007 52.6896) (width 0.3) (layer "B.Cu") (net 10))
 (segment (start 110.683 60.2292) (end 113.59 60.2292) (width 0.3) (layer "B.Cu") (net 1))
 (segment (start 116.355 51.501) (end 118.1155 51.501) (width 0.3) (layer "B.Cu") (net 1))
 (segment (start 116.02 51.1656) (end 111.553 51.1656) (width 0.3) (layer "B.Cu") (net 1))
 (segment (start 105.442 42.418) (end 106.553 42.418) (width 0.3) (layer "B.Cu") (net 1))
 (segment (start 106.553 42.418) (end 107.061 41.91) (width 0.3) (layer "B.Cu") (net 1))
 (segment (start 116.355 57.4638) (end 116.355 51.501) (width 0.3) (layer "B.Cu") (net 1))
 (segment (start 110.4955 57.15) (end 109.881 57.15) (width 0.3) (layer "B.Cu") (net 1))
 (segment (start 111.553 51.1656) (end 107.606 47.2185) (width 0.3) (layer "B.Cu") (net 1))
 (segment (start 109.475 59.0206) (end 110.683 60.2292) (width 0.3) (layer "B.Cu") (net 1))
 (segment (start 109.881 57.15) (end 109.352 57.6794) (width 0.3) (layer "B.Cu") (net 1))
 (segment (start 107.606 44.582) (end 105.442 42.418) (width 0.3) (layer "B.Cu") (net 1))
 (segment (start 109.352 57.6794) (end 109.352 58.4907) (width 0.3) (layer "B.Cu") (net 1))
 (segment (start 116.355 51.501) (end 116.02 51.1656) (width 0.3) (layer "B.Cu") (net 1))
 (segment (start 113.59 60.2292) (end 116.355 57.4638) (width 0.3) (layer "B.Cu") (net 1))
 (segment (start 109.352 58.4907) (end 109.475 58.6136) (width 0.3) (layer "B.Cu") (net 1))
 (segment (start 107.606 47.2185) (end 107.606 44.582) (width 0.3) (layer "B.Cu") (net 1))
 (segment (start 110.496 57.15) (end 110.4955 57.15) (width 0.3) (layer "B.Cu") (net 1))
 (segment (start 118.1155 51.501) (end 118.116 51.501) (width 0.3) (layer "B.Cu") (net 1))
 (segment (start 109.475 58.6136) (end 109.475 59.0206) (width 0.3) (layer "B.Cu") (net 1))
 (segment (start 105.442 42.418) (end 104.14 42.418) (width 0.3) (layer "B.Cu") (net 1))
 (segment (start 105.442 50.1729) (end 105.442 50.038) (width 0.3) (layer "F.Cu") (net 4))
 (segment (start 108.801 50.8) (end 106.069 50.8) (width 0.3) (layer "F.Cu") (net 4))
 (segment (start 111.269 52.2859) (end 110.727 51.7436) (width 0.3) (layer "F.Cu") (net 4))
 (segment (start 106.069 50.8) (end 105.442 50.1729) (width 0.3) (layer "F.Cu") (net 4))
 (segment (start 109.745 51.7436) (end 108.801 50.8) (width 0.3) (layer "F.Cu") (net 4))
 (segment (start 107.2515 57.15) (end 107.252 57.15) (width 0.3) (layer "F.Cu") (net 4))
 (segment (start 105.442 50.038) (end 104.14 50.038) (width 0.3) (layer "F.Cu") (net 4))
 (segment (start 110.727 51.7436) (end 109.745 51.7436) (width 0.3) (layer "F.Cu") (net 4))
 (segment (start 111.269 53.1323) (end 111.269 52.2859) (width 0.3) (layer "F.Cu") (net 4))
 (segment (start 107.252 57.15) (end 111.269 53.1323) (width 0.3) (layer "F.Cu") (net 4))
 (segment (start 123 49.53) (end 122.9995 49.53) (width 0.3) (layer "F.Cu") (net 11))
 (segment (start 122.9995 49.53) (end 121.035 49.53) (width 0.3) (layer "F.Cu") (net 11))
 (via (at 121.035 49.53) (size 0.8) (drill 0.4) (layers "F.Cu" "B.Cu") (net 11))
 (segment (start 120.3905 50.551) (end 120.3903 50.5508) (width 0.3) (layer "B.Cu") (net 11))
 (segment (start 121.035 49.9061) (end 121.035 49.53) (width 0.3) (layer "B.Cu") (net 11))
 (segment (start 120.3903 50.5508) (end 121.035 49.9061) (width 0.3) (layer "B.Cu") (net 11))
 (segment (start 120.39 50.551) (end 120.3903 50.5508) (width 0.3) (layer "B.Cu") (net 11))
 (segment (start 122.283 44.9367) (end 122.283 46.3374) (width 0.3) (layer "B.Cu") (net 17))
 (segment (start 122.987 44.2335) (end 122.283 44.9367) (width 0.3) (layer "B.Cu") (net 17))
 (segment (start 122.809 43.9795) (end 122.809 42.164) (width 0.3) (layer "B.Cu") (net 17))
 (segment (start 122.283 46.3374) (end 123.063 47.117) (width 0.3) (layer "B.Cu") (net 17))
 (segment (start 123.063 44.2335) (end 122.987 44.2335) (width 0.3) (layer "B.Cu") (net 17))
 (segment (start 123.063 44.2335) (end 122.809 43.9795) (width 0.3) (layer "B.Cu") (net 17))
 (segment (start 110.029 51.046) (end 108.513 49.53) (width 0.3) (layer "F.Cu") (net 6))
 (segment (start 113.068 62.7163) (end 113.0681 62.7162) (width 0.3) (layer "F.Cu") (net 6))
 (segment (start 113.068 63.2026) (end 109.889 63.2026) (width 0.3) (layer "F.Cu") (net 6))
 (segment (start 108.513 49.53) (end 107.252 49.53) (width 0.3) (layer "F.Cu") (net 6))
 (segment (start 113.068 62.7163) (end 113.068 63.2026) (width 0.3) (layer "F.Cu") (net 6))
 (segment (start 111.871 55.4495) (end 111.871 52.0366) (width 0.3) (layer "F.Cu") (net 6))
 (segment (start 107.2515 49.53) (end 107.252 49.53) (width 0.3) (layer "F.Cu") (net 6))
 (segment (start 109.657 57.6633) (end 111.871 55.4495) (width 0.3) (layer "F.Cu") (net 6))
 (segment (start 109.657 62.9713) (end 109.657 57.6633) (width 0.3) (layer "F.Cu") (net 6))
 (segment (start 113.068 62.23) (end 113.068 62.7163) (width 0.3) (layer "F.Cu") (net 6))
 (segment (start 111.871 52.0366) (end 110.88 51.046) (width 0.3) (layer "F.Cu") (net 6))
 (segment (start 110.88 51.046) (end 110.029 51.046) (width 0.3) (layer "F.Cu") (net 6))
 (segment (start 113.0681 62.7162) (end 113.0681 62.23) (width 0.3) (layer "F.Cu") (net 6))
 (segment (start 109.889 63.2026) (end 109.657 62.9713) (width 0.3) (layer "F.Cu") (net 6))
 (segment (start 106.756 61.2574) (end 106.756 61.7437) (width 0.3) (layer "F.Cu") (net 7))
 (segment (start 106.756 61.7437) (end 106.756 62.23) (width 0.3) (layer "F.Cu") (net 7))
 (segment (start 106.756 61.7437) (end 106.7562 61.7439) (width 0.3) (layer "F.Cu") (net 7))
 (segment (start 105.529 60.0299) (end 106.756 61.2574) (width 0.3) (layer "F.Cu") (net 7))
 (segment (start 106.7562 61.7439) (end 106.7562 62.23) (width 0.3) (layer "F.Cu") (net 7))
 (segment (start 107.2515 52.07) (end 107.2517 52.0702) (width 0.3) (layer "F.Cu") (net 7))
 (segment (start 105.529 53.7928) (end 105.529 60.0299) (width 0.3) (layer "F.Cu") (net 7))
 (segment (start 107.2517 52.0702) (end 105.529 53.7928) (width 0.3) (layer "F.Cu") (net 7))
 (segment (start 107.252 52.07) (end 107.2517 52.0702) (width 0.3) (layer "F.Cu") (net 7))
 (segment (start 123.4059 61.8947) (end 123.4059 62.23) (width 0.3) (layer "F.Cu") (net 8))
 (segment (start 123.406 61.8946) (end 123.4059 61.8947) (width 0.3) (layer "F.Cu") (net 8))
 (segment (start 123.406 61.8946) (end 123.406 62.23) (width 0.3) (layer "F.Cu") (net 8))
 (segment (start 123 57.15) (end 123.406 57.5564) (width 0.3) (layer "F.Cu") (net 8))
 (segment (start 123.406 57.5564) (end 123.406 61.8946) (width 0.3) (layer "F.Cu") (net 8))
 (segment (start 122.9995 57.15) (end 123 57.15) (width 0.3) (layer "F.Cu") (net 8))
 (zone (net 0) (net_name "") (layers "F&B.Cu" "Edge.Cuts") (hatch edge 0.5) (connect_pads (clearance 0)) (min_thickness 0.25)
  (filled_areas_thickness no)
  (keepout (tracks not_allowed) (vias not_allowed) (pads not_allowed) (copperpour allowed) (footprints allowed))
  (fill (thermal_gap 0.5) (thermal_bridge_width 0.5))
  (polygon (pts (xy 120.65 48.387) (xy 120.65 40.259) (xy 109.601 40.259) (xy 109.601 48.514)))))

